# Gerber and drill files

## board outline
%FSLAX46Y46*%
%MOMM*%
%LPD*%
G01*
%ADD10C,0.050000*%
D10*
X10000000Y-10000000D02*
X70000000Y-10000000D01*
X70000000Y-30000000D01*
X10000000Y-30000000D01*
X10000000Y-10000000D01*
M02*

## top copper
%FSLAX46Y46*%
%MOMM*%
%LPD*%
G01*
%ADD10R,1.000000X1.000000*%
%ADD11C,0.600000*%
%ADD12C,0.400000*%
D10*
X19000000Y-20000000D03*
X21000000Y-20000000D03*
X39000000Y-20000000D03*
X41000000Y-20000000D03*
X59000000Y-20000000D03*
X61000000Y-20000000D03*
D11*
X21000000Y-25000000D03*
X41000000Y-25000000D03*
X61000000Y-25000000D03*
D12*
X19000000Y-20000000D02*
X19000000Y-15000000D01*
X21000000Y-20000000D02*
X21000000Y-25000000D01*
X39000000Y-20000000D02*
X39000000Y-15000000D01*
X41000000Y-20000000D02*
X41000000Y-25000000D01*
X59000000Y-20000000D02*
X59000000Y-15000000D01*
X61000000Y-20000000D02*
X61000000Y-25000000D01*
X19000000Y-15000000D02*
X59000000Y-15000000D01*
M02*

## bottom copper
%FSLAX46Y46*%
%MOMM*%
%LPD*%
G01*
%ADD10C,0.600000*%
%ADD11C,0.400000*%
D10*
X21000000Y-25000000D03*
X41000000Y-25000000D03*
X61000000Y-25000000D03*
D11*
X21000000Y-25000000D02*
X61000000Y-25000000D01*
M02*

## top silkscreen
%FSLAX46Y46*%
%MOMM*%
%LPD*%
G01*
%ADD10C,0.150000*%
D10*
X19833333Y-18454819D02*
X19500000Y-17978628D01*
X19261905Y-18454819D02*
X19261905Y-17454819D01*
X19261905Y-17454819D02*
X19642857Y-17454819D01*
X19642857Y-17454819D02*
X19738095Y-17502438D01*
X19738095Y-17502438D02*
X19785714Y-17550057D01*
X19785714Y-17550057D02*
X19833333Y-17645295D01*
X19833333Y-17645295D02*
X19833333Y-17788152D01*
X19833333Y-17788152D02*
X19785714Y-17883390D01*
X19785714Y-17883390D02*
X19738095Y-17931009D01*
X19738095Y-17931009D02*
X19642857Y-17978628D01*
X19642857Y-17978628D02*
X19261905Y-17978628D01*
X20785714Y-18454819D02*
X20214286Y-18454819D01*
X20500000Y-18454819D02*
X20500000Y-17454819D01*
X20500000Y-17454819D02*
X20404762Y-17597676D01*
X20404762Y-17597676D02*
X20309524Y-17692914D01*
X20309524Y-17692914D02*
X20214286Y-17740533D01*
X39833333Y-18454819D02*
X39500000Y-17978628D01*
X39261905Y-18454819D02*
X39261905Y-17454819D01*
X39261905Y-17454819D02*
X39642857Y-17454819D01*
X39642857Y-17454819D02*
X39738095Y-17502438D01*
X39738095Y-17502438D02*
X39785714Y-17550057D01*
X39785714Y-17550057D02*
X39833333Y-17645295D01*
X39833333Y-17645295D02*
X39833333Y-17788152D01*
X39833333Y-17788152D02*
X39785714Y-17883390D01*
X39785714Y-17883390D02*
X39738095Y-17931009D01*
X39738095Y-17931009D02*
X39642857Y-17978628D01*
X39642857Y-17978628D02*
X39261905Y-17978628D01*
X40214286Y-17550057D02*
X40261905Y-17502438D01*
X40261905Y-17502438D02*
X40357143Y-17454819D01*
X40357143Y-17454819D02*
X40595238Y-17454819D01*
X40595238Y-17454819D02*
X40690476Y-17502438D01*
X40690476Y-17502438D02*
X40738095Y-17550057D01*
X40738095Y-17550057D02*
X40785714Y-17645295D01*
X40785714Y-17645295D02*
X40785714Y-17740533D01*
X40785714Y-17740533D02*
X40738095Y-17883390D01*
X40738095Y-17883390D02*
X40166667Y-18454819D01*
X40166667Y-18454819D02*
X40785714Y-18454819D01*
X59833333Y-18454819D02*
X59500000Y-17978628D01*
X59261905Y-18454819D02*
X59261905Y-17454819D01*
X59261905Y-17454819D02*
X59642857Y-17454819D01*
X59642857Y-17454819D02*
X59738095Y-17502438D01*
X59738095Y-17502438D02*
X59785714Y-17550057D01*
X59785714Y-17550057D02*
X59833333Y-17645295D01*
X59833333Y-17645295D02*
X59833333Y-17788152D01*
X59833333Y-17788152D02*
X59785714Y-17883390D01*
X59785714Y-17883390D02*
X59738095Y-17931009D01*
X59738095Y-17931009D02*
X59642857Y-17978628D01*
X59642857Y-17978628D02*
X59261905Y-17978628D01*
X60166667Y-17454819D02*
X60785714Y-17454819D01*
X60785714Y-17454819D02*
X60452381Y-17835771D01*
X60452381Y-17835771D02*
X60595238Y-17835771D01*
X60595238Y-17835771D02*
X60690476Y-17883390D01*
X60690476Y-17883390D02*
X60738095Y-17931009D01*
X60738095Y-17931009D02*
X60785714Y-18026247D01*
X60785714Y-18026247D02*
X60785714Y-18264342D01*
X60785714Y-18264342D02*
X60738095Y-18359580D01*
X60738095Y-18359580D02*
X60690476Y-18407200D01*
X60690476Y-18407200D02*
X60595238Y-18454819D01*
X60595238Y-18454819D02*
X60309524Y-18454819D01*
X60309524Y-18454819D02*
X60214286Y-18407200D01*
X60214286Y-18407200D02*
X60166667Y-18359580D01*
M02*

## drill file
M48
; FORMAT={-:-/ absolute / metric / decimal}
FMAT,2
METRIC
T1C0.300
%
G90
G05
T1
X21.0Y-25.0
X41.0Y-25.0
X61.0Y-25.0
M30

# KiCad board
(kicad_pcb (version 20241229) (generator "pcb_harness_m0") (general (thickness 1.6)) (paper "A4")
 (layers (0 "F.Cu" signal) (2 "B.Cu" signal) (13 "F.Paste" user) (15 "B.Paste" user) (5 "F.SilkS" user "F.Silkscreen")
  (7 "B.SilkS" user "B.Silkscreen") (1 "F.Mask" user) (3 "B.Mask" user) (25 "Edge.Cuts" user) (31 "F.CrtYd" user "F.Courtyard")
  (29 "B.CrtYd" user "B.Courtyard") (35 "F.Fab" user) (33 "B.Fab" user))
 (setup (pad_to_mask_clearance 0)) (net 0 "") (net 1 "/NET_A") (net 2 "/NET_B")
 (gr_rect (start 10 10) (end 70 30) (stroke (width 0.05) (type default)) (fill none) (layer "Edge.Cuts"))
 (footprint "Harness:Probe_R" (layer "F.Cu") (at 20 20)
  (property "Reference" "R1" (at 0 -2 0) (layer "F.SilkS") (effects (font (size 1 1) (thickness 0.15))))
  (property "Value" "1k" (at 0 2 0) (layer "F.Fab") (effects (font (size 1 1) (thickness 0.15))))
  (pad "1" smd rect (at -1 0) (size 1 1) (layers "F.Cu" "F.Paste" "F.Mask") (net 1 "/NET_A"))
  (pad "2" smd rect (at 1 0) (size 1 1) (layers "F.Cu" "F.Paste" "F.Mask") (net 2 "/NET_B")))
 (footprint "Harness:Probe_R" (layer "F.Cu") (at 40 20)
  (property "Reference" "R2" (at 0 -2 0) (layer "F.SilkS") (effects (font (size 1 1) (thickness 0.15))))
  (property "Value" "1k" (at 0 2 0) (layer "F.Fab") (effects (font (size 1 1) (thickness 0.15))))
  (pad "1" smd rect (at -1 0) (size 1 1) (layers "F.Cu" "F.Paste" "F.Mask") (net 1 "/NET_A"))
  (pad "2" smd rect (at 1 0) (size 1 1) (layers "F.Cu" "F.Paste" "F.Mask") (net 2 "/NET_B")))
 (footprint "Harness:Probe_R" (layer "F.Cu") (at 60 20)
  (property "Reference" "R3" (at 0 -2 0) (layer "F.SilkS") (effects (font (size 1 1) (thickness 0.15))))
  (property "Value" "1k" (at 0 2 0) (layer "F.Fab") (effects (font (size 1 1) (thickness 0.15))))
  (pad "1" smd rect (at -1 0) (size 1 1) (layers "F.Cu" "F.Paste" "F.Mask") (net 1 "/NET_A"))
  (pad "2" smd rect (at 1 0) (size 1 1) (layers "F.Cu" "F.Paste" "F.Mask") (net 2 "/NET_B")))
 (segment (start 19 20) (end 19 15) (width 0.4) (layer "F.Cu") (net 1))
 (segment (start 21 20) (end 21 25) (width 0.4) (layer "F.Cu") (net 2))
 (via (at 21 25) (size 0.6) (drill 0.3) (layers "F.Cu" "B.Cu") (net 2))
 (segment (start 39 20) (end 39 15) (width 0.4) (layer "F.Cu") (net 1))
 (segment (start 41 20) (end 41 25) (width 0.4) (layer "F.Cu") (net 2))
 (via (at 41 25) (size 0.6) (drill 0.3) (layers "F.Cu" "B.Cu") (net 2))
 (segment (start 59 20) (end 59 15) (width 0.4) (layer "F.Cu") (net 1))
 (segment (start 61 20) (end 61 25) (width 0.4) (layer "F.Cu") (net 2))
 (via (at 61 25) (size 0.6) (drill 0.3) (layers "F.Cu" "B.Cu") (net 2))
 (segment (start 19 15) (end 59 15) (width 0.4) (layer "F.Cu") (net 1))
 (segment (start 21 25) (end 61 25) (width 0.4) (layer "B.Cu") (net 2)))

